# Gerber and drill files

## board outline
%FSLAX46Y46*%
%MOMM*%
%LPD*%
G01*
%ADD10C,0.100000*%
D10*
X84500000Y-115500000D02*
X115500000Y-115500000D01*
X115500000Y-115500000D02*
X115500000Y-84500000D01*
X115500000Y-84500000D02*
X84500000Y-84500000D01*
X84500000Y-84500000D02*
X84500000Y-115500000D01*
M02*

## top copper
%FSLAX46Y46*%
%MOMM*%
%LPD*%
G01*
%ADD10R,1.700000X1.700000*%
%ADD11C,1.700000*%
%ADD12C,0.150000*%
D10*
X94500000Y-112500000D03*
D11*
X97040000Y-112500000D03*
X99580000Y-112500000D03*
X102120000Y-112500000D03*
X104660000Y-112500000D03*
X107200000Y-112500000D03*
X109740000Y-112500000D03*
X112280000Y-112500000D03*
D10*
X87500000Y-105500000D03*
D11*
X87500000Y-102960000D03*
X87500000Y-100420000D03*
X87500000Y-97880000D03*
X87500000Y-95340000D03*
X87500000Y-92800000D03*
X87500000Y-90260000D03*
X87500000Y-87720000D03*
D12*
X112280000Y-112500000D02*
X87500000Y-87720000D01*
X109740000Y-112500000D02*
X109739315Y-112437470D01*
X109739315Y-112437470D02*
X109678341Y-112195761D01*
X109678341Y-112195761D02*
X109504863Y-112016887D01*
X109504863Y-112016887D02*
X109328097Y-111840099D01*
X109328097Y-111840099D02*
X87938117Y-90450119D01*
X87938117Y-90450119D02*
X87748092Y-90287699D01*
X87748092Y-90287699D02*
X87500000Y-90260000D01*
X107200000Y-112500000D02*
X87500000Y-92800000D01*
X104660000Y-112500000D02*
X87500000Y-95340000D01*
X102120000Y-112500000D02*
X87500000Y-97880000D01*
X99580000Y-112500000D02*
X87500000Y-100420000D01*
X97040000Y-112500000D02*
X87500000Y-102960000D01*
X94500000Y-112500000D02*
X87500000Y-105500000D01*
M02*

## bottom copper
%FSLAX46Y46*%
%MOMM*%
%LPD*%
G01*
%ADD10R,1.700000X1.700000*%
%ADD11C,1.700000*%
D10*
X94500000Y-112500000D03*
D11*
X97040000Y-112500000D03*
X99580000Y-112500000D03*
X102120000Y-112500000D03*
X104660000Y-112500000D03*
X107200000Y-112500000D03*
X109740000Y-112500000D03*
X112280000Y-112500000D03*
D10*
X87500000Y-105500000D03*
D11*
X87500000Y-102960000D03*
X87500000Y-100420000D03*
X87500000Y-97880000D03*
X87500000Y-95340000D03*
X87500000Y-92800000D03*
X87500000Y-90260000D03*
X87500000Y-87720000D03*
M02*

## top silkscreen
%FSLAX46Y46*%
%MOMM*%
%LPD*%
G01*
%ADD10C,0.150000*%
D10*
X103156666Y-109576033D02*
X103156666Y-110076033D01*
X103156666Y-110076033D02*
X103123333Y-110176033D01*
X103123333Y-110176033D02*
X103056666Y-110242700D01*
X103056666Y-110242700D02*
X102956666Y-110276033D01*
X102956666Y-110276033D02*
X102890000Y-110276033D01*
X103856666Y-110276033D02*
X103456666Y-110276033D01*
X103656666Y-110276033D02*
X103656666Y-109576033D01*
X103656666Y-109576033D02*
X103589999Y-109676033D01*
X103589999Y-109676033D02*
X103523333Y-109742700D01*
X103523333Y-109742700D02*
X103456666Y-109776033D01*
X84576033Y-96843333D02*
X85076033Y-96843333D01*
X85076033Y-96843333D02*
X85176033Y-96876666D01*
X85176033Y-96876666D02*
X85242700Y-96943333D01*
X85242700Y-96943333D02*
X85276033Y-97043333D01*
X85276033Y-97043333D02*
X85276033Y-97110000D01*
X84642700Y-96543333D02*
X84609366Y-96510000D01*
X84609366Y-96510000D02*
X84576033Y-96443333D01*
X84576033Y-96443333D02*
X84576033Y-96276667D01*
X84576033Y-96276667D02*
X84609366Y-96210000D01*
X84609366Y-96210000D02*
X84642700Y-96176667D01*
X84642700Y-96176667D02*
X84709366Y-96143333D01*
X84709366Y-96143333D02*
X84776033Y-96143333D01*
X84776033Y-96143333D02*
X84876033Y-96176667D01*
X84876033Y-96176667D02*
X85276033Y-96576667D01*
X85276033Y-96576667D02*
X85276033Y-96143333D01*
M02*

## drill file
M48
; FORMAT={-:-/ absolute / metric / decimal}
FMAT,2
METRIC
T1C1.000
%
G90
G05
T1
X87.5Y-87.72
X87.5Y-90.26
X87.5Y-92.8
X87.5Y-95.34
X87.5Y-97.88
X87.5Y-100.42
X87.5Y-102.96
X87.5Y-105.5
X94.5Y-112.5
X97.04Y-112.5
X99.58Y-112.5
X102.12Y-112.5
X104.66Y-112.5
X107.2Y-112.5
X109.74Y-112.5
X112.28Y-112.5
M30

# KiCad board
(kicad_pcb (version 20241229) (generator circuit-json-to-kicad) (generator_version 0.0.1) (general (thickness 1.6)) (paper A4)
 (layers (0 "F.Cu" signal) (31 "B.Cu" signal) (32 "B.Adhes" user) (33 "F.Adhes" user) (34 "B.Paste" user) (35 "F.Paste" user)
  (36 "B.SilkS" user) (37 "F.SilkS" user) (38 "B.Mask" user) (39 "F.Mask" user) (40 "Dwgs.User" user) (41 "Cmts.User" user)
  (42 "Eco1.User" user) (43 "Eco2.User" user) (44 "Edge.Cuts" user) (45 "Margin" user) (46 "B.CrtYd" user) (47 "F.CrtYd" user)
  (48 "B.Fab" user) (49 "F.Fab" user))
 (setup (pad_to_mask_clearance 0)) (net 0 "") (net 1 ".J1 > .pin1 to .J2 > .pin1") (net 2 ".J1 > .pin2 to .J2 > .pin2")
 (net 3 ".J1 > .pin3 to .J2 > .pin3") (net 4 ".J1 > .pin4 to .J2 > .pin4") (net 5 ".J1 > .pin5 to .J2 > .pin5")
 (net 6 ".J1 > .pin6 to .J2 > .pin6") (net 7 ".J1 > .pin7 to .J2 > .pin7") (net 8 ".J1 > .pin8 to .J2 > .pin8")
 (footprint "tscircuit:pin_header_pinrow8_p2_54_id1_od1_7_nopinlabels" (layer F.Cu) (at 103.39 112.5 0)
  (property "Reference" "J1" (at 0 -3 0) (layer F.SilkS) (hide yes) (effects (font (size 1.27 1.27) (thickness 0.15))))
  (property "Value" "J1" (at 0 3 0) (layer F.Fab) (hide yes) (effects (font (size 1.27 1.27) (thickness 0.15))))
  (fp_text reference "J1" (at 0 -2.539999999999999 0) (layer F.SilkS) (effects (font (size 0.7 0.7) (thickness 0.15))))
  (pad "1" thru_hole rect (at -8.89 0 0) (size 1.7 1.7) (drill 1) (layers *.Cu *.Mask) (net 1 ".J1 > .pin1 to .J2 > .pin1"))
  (pad "2" thru_hole circle (at -6.3500000000000005 0 0) (size 1.7 1.7) (drill 1) (layers *.Cu *.Mask) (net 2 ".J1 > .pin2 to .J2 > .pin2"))
  (pad "3" thru_hole circle (at -3.8100000000000005 0 0) (size 1.7 1.7) (drill 1) (layers *.Cu *.Mask) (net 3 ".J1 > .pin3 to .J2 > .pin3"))
  (pad "4" thru_hole circle (at -1.2700000000000005 0 0) (size 1.7 1.7) (drill 1) (layers *.Cu *.Mask) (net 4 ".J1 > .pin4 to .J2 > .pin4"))
  (pad "5" thru_hole circle (at 1.27 0 0) (size 1.7 1.7) (drill 1) (layers *.Cu *.Mask) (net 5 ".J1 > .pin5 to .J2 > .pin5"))
  (pad "6" thru_hole circle (at 3.809999999999999 0 0) (size 1.7 1.7) (drill 1) (layers *.Cu *.Mask) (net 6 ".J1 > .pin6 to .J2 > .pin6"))
  (pad "7" thru_hole circle (at 6.35 0 0) (size 1.7 1.7) (drill 1) (layers *.Cu *.Mask) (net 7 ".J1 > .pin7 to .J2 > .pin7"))
  (pad "8" thru_hole circle (at 8.89 0 0) (size 1.7 1.7) (drill 1) (layers *.Cu *.Mask) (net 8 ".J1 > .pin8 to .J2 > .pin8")))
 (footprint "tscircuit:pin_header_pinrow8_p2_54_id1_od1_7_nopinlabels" (layer F.Cu) (at 87.5 96.61 90)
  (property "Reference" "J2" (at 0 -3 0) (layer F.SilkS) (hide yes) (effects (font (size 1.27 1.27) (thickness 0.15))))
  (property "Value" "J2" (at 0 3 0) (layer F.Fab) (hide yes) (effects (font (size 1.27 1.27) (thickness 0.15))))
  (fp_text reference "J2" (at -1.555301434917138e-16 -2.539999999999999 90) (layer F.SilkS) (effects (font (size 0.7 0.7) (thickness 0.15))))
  (pad "1" thru_hole rect (at -8.89 5.443555022209985e-16 90) (size 1.7 1.7) (drill 1) (layers *.Cu *.Mask)
   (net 1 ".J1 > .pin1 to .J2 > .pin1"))
  (pad "2" thru_hole circle (at -6.3500000000000005 3.8882535872928466e-16 0) (size 1.7 1.7) (drill 1) (layers *.Cu *.Mask)
   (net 2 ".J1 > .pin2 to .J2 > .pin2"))
  (pad "3" thru_hole circle (at -3.8100000000000005 2.332952152375708e-16 0) (size 1.7 1.7) (drill 1) (layers *.Cu *.Mask)
   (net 3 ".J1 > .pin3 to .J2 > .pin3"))
  (pad "4" thru_hole circle (at -1.2700000000000005 7.776507174585695e-17 0) (size 1.7 1.7) (drill 1) (layers *.Cu *.Mask)
   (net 4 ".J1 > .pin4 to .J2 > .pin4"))
  (pad "5" thru_hole circle (at 1.27 -7.776507174585693e-17 0) (size 1.7 1.7) (drill 1) (layers *.Cu *.Mask)
   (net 5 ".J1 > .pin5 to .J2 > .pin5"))
  (pad "6" thru_hole circle (at 3.809999999999999 -2.3329521523757073e-16 0) (size 1.7 1.7) (drill 1) (layers *.Cu *.Mask)
   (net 6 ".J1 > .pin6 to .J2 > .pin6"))
  (pad "7" thru_hole circle (at 6.35 -3.888253587292846e-16 0) (size 1.7 1.7) (drill 1) (layers *.Cu *.Mask)
   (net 7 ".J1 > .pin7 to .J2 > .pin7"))
  (pad "8" thru_hole circle (at 8.89 -5.443555022209985e-16 0) (size 1.7 1.7) (drill 1) (layers *.Cu *.Mask)
   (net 8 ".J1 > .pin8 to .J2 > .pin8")))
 (segment (start 112.28 112.5) (end 87.5 87.72) (width 0.15) (layer F.Cu) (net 8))
 (segment (start 109.74 112.5) (end 109.73931521955309 112.43746996820214) (width 0.15) (layer F.Cu) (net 7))
 (segment (start 109.73931521955309 112.43746996820214) (end 109.6783409397556 112.19576112126337) (width 0.15) (layer F.Cu) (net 7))
 (segment (start 109.6783409397556 112.19576112126337) (end 109.5048627412114 112.01688657817145) (width 0.15) (layer F.Cu) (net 7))
 (segment (start 109.5048627412114 112.01688657817145) (end 109.32809727104033 111.84009868483874) (width 0.15) (layer F.Cu) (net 7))
 (segment (start 109.32809727104033 111.84009868483874) (end 87.93811714014728 90.45011855394567) (width 0.15) (layer F.Cu) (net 7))
 (segment (start 87.93811714014728 90.45011855394567) (end 87.74809175010869 90.28769914930984) (width 0.15) (layer F.Cu) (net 7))
 (segment (start 87.74809175010869 90.28769914930984) (end 87.5 90.26) (width 0.15) (layer F.Cu) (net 7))
 (segment (start 107.2 112.5) (end 87.5 92.8) (width 0.15) (layer F.Cu) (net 6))
 (segment (start 104.66 112.5) (end 87.5 95.34) (width 0.15) (layer F.Cu) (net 5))
 (segment (start 102.12 112.5) (end 87.5 97.88) (width 0.15) (layer F.Cu) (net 4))
 (segment (start 99.58 112.5) (end 87.5 100.42) (width 0.15) (layer F.Cu) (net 3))
 (segment (start 97.04 112.5) (end 87.5 102.96) (width 0.15) (layer F.Cu) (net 2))
 (segment (start 94.5 112.5) (end 87.5 105.5) (width 0.15) (layer F.Cu) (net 1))
 (gr_line (start 84.5 115.5) (end 115.5 115.5) (width 0.1) (layer Edge.Cuts))
 (gr_line (start 115.5 115.5) (end 115.5 84.5) (width 0.1) (layer Edge.Cuts))
 (gr_line (start 115.5 84.5) (end 84.5 84.5) (width 0.1) (layer Edge.Cuts))
 (gr_line (start 84.5 84.5) (end 84.5 115.5) (width 0.1) (layer Edge.Cuts)))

